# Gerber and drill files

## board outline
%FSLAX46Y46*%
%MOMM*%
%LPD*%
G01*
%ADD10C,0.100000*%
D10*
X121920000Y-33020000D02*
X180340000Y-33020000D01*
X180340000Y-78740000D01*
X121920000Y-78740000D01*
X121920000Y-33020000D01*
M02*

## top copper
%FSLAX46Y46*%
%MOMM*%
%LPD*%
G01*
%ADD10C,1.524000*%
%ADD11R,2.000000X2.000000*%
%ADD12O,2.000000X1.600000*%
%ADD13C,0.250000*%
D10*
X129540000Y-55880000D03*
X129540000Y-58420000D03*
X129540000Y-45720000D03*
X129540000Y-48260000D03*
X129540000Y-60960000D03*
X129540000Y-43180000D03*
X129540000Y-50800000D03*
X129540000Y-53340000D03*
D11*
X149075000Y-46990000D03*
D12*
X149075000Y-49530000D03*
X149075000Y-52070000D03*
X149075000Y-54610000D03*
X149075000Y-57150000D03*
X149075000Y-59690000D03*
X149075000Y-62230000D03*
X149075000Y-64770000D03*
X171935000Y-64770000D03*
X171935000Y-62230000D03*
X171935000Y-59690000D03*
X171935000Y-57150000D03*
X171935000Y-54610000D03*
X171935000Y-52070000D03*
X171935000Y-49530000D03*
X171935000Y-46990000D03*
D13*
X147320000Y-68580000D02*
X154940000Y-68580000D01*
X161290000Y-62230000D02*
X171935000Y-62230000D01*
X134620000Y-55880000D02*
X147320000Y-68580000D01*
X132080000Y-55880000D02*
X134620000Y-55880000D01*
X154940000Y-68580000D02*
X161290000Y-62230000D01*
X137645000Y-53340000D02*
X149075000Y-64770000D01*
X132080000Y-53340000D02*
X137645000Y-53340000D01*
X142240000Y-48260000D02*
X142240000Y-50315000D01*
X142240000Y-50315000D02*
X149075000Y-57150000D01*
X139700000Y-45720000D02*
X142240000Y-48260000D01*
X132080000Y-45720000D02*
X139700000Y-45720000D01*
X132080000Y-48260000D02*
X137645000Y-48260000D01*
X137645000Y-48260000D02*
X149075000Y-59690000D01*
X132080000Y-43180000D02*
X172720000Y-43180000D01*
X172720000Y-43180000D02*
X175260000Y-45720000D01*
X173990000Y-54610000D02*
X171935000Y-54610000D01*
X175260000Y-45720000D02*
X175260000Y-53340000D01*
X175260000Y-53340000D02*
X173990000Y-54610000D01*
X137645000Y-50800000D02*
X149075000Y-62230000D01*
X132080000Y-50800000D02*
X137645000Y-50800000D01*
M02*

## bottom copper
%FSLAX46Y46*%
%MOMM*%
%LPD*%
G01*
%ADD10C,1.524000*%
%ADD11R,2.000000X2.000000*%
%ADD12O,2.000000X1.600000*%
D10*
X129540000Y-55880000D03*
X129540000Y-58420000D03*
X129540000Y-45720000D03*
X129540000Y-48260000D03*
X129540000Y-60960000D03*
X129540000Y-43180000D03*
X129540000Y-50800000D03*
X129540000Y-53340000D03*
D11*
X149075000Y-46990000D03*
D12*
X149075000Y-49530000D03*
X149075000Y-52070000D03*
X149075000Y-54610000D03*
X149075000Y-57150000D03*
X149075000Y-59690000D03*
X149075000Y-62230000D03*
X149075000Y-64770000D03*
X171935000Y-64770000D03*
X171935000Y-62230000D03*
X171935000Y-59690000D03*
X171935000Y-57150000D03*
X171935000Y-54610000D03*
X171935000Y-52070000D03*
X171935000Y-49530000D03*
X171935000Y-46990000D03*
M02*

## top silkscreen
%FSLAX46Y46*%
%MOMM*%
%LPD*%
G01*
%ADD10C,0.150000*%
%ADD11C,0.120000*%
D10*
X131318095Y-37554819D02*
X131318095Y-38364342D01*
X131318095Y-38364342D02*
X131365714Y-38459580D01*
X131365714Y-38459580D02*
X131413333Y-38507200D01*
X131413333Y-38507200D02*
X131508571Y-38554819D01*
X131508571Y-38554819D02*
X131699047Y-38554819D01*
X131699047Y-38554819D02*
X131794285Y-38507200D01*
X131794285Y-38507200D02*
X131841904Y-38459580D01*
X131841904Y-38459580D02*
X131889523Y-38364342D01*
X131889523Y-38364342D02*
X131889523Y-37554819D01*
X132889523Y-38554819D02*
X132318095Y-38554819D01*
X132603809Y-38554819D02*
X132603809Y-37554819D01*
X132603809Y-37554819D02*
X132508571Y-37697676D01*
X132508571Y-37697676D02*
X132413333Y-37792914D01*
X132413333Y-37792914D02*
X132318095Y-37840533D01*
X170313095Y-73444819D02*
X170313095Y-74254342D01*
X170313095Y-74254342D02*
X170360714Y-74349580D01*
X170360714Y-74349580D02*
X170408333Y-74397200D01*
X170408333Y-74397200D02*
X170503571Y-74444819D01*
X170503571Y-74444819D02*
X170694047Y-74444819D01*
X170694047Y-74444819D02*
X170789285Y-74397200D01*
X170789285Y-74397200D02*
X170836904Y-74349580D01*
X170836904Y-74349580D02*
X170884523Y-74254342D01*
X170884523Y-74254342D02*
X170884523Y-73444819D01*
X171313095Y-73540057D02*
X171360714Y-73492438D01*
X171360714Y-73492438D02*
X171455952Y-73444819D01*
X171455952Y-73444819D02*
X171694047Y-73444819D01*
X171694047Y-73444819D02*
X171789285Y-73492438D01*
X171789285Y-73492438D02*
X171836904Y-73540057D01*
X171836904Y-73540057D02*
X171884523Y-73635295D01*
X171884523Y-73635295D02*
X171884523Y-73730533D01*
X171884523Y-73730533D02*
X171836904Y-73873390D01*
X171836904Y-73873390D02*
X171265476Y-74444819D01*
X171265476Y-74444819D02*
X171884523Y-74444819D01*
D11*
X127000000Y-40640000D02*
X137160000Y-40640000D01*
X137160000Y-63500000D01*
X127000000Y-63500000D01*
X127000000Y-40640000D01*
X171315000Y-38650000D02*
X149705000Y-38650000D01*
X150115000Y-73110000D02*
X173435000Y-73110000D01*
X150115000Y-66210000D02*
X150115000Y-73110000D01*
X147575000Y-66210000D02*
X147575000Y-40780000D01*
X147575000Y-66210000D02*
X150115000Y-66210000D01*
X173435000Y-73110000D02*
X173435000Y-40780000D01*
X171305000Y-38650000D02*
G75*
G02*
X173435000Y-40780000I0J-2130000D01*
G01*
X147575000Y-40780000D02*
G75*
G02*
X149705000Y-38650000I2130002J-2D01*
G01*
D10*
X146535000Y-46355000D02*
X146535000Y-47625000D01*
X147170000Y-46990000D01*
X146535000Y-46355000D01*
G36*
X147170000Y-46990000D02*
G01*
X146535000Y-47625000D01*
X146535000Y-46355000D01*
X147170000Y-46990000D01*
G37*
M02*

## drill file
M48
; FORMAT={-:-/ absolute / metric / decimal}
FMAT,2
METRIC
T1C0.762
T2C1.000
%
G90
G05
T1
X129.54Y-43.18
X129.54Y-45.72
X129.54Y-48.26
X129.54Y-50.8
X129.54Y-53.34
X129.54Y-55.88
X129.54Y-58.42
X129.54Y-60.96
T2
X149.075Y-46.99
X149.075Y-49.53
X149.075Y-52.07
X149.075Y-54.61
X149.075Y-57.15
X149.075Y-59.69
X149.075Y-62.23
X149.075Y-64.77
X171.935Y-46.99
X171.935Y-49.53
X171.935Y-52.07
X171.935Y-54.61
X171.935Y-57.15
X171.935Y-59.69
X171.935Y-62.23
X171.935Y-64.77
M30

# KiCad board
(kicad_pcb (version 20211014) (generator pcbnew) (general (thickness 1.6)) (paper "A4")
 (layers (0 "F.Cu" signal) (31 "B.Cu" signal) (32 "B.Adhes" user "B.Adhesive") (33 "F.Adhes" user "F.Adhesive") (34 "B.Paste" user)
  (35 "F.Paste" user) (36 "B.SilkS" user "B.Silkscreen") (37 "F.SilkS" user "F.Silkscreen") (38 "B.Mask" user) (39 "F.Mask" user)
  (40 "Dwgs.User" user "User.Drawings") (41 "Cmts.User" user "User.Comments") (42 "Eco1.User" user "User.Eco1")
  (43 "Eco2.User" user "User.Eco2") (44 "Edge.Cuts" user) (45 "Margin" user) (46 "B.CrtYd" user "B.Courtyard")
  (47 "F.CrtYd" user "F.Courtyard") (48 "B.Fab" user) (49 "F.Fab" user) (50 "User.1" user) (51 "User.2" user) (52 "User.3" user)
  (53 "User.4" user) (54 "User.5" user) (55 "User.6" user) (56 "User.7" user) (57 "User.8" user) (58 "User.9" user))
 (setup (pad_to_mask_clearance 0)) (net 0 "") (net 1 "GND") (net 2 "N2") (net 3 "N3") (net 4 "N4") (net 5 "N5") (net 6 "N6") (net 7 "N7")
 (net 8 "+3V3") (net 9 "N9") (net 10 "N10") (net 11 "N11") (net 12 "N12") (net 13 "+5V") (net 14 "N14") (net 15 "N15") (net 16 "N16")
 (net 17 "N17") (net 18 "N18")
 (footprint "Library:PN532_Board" (layer "F.Cu") (at 132.08 53.34)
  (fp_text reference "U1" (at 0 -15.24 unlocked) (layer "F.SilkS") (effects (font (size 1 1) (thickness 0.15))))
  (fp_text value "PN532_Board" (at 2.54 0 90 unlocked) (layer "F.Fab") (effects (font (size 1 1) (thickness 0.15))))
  (fp_rect (start -5.08 -12.7) (end 5.08 10.16) (layer "F.SilkS") (width 0.12) (fill none))
  (pad "GND" thru_hole circle (at -2.54 2.54) (size 1.524 1.524) (drill 0.762) (layers *.Cu *.Mask) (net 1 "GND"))
  (pad "IRQ" thru_hole circle (at -2.54 5.08) (size 1.524 1.524) (drill 0.762) (layers *.Cu *.Mask) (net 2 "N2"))
  (pad "MISO" thru_hole circle (at -2.54 -7.62) (size 1.524 1.524) (drill 0.762) (layers *.Cu *.Mask) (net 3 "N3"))
  (pad "MOSI" thru_hole circle (at -2.54 -5.08) (size 1.524 1.524) (drill 0.762) (layers *.Cu *.Mask) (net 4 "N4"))
  (pad "RSTO" thru_hole circle (at -2.54 7.62) (size 1.524 1.524) (drill 0.762) (layers *.Cu *.Mask) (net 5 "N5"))
  (pad "SCK" thru_hole circle (at -2.54 -10.16) (size 1.524 1.524) (drill 0.762) (layers *.Cu *.Mask) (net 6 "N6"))
  (pad "SS" thru_hole circle (at -2.54 -2.54) (size 1.524 1.524) (drill 0.762) (layers *.Cu *.Mask) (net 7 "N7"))
  (pad "VCC" thru_hole circle (at -2.54 0) (size 1.524 1.524) (drill 0.762) (layers *.Cu *.Mask) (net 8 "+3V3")))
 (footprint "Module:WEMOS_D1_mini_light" (layer "F.Cu") (at 149.075 46.99)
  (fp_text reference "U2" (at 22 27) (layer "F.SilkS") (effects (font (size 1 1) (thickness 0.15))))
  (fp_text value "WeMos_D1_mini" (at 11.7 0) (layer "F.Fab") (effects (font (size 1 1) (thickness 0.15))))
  (fp_line (start 22.24 -8.34) (end 0.63 -8.34) (layer "F.SilkS") (width 0.12))
  (fp_line (start 1.04 26.12) (end 24.36 26.12) (layer "F.SilkS") (width 0.12))
  (fp_line (start 1.04 19.22) (end 1.04 26.12) (layer "F.SilkS") (width 0.12))
  (fp_line (start -1.5 19.22) (end -1.5 -6.21) (layer "F.SilkS") (width 0.12))
  (fp_line (start -1.5 19.22) (end 1.04 19.22) (layer "F.SilkS") (width 0.12))
  (fp_line (start 24.36 26.12) (end 24.36 -6.21) (layer "F.SilkS") (width 0.12))
  (fp_arc (start 22.23 -8.34) (mid 23.736137 -7.716137) (end 24.36 -6.21) (layer "F.SilkS") (width 0.12))
  (fp_arc (start -1.5 -6.21) (mid -0.876137 -7.716137) (end 0.63 -8.34) (layer "F.SilkS") (width 0.12))
  (fp_poly (pts (xy -2.54 -0.635) (xy -2.54 0.635) (xy -1.905 0)) (layer "F.SilkS") (width 0.15) (fill solid))
  (pad "1" thru_hole rect (at 0 0) (size 2 2) (drill 1) (layers *.Cu *.Mask) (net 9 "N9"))
  (pad "2" thru_hole oval (at 0 2.54) (size 2 1.6) (drill 1) (layers *.Cu *.Mask) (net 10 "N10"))
  (pad "3" thru_hole oval (at 0 5.08) (size 2 1.6) (drill 1) (layers *.Cu *.Mask) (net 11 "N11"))
  (pad "4" thru_hole oval (at 0 7.62) (size 2 1.6) (drill 1) (layers *.Cu *.Mask) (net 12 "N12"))
  (pad "5" thru_hole oval (at 0 10.16) (size 2 1.6) (drill 1) (layers *.Cu *.Mask) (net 3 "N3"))
  (pad "6" thru_hole oval (at 0 12.7) (size 2 1.6) (drill 1) (layers *.Cu *.Mask) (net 4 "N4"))
  (pad "7" thru_hole oval (at 0 15.24) (size 2 1.6) (drill 1) (layers *.Cu *.Mask) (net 7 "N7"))
  (pad "8" thru_hole oval (at 0 17.78) (size 2 1.6) (drill 1) (layers *.Cu *.Mask) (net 8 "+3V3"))
  (pad "9" thru_hole oval (at 22.86 17.78) (size 2 1.6) (drill 1) (layers *.Cu *.Mask) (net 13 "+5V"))
  (pad "10" thru_hole oval (at 22.86 15.24) (size 2 1.6) (drill 1) (layers *.Cu *.Mask) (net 1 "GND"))
  (pad "11" thru_hole oval (at 22.86 12.7) (size 2 1.6) (drill 1) (layers *.Cu *.Mask) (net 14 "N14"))
  (pad "12" thru_hole oval (at 22.86 10.16) (size 2 1.6) (drill 1) (layers *.Cu *.Mask) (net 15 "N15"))
  (pad "13" thru_hole oval (at 22.86 7.62) (size 2 1.6) (drill 1) (layers *.Cu *.Mask) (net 6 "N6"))
  (pad "14" thru_hole oval (at 22.86 5.08) (size 2 1.6) (drill 1) (layers *.Cu *.Mask) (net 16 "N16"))
  (pad "15" thru_hole oval (at 22.86 2.54) (size 2 1.6) (drill 1) (layers *.Cu *.Mask) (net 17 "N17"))
  (pad "16" thru_hole oval (at 22.86 0) (size 2 1.6) (drill 1) (layers *.Cu *.Mask) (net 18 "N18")))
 (gr_rect (start 121.92 33.02) (end 180.34 78.74) (layer "Edge.Cuts") (width 0.1) (fill none))
 (segment (start 147.32 68.58) (end 154.94 68.58) (width 0.25) (layer "F.Cu") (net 1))
 (segment (start 161.29 62.23) (end 171.935 62.23) (width 0.25) (layer "F.Cu") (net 1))
 (segment (start 134.62 55.88) (end 147.32 68.58) (width 0.25) (layer "F.Cu") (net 1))
 (segment (start 132.08 55.88) (end 134.62 55.88) (width 0.25) (layer "F.Cu") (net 1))
 (segment (start 154.94 68.58) (end 161.29 62.23) (width 0.25) (layer "F.Cu") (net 1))
 (segment (start 137.645 53.34) (end 149.075 64.77) (width 0.25) (layer "F.Cu") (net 8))
 (segment (start 132.08 53.34) (end 137.645 53.34) (width 0.25) (layer "F.Cu") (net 8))
 (segment (start 142.24 48.26) (end 142.24 50.315) (width 0.25) (layer "F.Cu") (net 3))
 (segment (start 142.24 50.315) (end 149.075 57.15) (width 0.25) (layer "F.Cu") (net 3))
 (segment (start 139.7 45.72) (end 142.24 48.26) (width 0.25) (layer "F.Cu") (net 3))
 (segment (start 132.08 45.72) (end 139.7 45.72) (width 0.25) (layer "F.Cu") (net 3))
 (segment (start 132.08 48.26) (end 137.645 48.26) (width 0.25) (layer "F.Cu") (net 4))
 (segment (start 137.645 48.26) (end 149.075 59.69) (width 0.25) (layer "F.Cu") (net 4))
 (segment (start 132.08 43.18) (end 172.72 43.18) (width 0.25) (layer "F.Cu") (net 6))
 (segment (start 172.72 43.18) (end 175.26 45.72) (width 0.25) (layer "F.Cu") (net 6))
 (segment (start 173.99 54.61) (end 171.935 54.61) (width 0.25) (layer "F.Cu") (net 6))
 (segment (start 175.26 45.72) (end 175.26 53.34) (width 0.25) (layer "F.Cu") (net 6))
 (segment (start 175.26 53.34) (end 173.99 54.61) (width 0.25) (layer "F.Cu") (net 6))
 (segment (start 137.645 50.8) (end 149.075 62.23) (width 0.25) (layer "F.Cu") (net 7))
 (segment (start 132.08 50.8) (end 137.645 50.8) (width 0.25) (layer "F.Cu") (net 7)))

